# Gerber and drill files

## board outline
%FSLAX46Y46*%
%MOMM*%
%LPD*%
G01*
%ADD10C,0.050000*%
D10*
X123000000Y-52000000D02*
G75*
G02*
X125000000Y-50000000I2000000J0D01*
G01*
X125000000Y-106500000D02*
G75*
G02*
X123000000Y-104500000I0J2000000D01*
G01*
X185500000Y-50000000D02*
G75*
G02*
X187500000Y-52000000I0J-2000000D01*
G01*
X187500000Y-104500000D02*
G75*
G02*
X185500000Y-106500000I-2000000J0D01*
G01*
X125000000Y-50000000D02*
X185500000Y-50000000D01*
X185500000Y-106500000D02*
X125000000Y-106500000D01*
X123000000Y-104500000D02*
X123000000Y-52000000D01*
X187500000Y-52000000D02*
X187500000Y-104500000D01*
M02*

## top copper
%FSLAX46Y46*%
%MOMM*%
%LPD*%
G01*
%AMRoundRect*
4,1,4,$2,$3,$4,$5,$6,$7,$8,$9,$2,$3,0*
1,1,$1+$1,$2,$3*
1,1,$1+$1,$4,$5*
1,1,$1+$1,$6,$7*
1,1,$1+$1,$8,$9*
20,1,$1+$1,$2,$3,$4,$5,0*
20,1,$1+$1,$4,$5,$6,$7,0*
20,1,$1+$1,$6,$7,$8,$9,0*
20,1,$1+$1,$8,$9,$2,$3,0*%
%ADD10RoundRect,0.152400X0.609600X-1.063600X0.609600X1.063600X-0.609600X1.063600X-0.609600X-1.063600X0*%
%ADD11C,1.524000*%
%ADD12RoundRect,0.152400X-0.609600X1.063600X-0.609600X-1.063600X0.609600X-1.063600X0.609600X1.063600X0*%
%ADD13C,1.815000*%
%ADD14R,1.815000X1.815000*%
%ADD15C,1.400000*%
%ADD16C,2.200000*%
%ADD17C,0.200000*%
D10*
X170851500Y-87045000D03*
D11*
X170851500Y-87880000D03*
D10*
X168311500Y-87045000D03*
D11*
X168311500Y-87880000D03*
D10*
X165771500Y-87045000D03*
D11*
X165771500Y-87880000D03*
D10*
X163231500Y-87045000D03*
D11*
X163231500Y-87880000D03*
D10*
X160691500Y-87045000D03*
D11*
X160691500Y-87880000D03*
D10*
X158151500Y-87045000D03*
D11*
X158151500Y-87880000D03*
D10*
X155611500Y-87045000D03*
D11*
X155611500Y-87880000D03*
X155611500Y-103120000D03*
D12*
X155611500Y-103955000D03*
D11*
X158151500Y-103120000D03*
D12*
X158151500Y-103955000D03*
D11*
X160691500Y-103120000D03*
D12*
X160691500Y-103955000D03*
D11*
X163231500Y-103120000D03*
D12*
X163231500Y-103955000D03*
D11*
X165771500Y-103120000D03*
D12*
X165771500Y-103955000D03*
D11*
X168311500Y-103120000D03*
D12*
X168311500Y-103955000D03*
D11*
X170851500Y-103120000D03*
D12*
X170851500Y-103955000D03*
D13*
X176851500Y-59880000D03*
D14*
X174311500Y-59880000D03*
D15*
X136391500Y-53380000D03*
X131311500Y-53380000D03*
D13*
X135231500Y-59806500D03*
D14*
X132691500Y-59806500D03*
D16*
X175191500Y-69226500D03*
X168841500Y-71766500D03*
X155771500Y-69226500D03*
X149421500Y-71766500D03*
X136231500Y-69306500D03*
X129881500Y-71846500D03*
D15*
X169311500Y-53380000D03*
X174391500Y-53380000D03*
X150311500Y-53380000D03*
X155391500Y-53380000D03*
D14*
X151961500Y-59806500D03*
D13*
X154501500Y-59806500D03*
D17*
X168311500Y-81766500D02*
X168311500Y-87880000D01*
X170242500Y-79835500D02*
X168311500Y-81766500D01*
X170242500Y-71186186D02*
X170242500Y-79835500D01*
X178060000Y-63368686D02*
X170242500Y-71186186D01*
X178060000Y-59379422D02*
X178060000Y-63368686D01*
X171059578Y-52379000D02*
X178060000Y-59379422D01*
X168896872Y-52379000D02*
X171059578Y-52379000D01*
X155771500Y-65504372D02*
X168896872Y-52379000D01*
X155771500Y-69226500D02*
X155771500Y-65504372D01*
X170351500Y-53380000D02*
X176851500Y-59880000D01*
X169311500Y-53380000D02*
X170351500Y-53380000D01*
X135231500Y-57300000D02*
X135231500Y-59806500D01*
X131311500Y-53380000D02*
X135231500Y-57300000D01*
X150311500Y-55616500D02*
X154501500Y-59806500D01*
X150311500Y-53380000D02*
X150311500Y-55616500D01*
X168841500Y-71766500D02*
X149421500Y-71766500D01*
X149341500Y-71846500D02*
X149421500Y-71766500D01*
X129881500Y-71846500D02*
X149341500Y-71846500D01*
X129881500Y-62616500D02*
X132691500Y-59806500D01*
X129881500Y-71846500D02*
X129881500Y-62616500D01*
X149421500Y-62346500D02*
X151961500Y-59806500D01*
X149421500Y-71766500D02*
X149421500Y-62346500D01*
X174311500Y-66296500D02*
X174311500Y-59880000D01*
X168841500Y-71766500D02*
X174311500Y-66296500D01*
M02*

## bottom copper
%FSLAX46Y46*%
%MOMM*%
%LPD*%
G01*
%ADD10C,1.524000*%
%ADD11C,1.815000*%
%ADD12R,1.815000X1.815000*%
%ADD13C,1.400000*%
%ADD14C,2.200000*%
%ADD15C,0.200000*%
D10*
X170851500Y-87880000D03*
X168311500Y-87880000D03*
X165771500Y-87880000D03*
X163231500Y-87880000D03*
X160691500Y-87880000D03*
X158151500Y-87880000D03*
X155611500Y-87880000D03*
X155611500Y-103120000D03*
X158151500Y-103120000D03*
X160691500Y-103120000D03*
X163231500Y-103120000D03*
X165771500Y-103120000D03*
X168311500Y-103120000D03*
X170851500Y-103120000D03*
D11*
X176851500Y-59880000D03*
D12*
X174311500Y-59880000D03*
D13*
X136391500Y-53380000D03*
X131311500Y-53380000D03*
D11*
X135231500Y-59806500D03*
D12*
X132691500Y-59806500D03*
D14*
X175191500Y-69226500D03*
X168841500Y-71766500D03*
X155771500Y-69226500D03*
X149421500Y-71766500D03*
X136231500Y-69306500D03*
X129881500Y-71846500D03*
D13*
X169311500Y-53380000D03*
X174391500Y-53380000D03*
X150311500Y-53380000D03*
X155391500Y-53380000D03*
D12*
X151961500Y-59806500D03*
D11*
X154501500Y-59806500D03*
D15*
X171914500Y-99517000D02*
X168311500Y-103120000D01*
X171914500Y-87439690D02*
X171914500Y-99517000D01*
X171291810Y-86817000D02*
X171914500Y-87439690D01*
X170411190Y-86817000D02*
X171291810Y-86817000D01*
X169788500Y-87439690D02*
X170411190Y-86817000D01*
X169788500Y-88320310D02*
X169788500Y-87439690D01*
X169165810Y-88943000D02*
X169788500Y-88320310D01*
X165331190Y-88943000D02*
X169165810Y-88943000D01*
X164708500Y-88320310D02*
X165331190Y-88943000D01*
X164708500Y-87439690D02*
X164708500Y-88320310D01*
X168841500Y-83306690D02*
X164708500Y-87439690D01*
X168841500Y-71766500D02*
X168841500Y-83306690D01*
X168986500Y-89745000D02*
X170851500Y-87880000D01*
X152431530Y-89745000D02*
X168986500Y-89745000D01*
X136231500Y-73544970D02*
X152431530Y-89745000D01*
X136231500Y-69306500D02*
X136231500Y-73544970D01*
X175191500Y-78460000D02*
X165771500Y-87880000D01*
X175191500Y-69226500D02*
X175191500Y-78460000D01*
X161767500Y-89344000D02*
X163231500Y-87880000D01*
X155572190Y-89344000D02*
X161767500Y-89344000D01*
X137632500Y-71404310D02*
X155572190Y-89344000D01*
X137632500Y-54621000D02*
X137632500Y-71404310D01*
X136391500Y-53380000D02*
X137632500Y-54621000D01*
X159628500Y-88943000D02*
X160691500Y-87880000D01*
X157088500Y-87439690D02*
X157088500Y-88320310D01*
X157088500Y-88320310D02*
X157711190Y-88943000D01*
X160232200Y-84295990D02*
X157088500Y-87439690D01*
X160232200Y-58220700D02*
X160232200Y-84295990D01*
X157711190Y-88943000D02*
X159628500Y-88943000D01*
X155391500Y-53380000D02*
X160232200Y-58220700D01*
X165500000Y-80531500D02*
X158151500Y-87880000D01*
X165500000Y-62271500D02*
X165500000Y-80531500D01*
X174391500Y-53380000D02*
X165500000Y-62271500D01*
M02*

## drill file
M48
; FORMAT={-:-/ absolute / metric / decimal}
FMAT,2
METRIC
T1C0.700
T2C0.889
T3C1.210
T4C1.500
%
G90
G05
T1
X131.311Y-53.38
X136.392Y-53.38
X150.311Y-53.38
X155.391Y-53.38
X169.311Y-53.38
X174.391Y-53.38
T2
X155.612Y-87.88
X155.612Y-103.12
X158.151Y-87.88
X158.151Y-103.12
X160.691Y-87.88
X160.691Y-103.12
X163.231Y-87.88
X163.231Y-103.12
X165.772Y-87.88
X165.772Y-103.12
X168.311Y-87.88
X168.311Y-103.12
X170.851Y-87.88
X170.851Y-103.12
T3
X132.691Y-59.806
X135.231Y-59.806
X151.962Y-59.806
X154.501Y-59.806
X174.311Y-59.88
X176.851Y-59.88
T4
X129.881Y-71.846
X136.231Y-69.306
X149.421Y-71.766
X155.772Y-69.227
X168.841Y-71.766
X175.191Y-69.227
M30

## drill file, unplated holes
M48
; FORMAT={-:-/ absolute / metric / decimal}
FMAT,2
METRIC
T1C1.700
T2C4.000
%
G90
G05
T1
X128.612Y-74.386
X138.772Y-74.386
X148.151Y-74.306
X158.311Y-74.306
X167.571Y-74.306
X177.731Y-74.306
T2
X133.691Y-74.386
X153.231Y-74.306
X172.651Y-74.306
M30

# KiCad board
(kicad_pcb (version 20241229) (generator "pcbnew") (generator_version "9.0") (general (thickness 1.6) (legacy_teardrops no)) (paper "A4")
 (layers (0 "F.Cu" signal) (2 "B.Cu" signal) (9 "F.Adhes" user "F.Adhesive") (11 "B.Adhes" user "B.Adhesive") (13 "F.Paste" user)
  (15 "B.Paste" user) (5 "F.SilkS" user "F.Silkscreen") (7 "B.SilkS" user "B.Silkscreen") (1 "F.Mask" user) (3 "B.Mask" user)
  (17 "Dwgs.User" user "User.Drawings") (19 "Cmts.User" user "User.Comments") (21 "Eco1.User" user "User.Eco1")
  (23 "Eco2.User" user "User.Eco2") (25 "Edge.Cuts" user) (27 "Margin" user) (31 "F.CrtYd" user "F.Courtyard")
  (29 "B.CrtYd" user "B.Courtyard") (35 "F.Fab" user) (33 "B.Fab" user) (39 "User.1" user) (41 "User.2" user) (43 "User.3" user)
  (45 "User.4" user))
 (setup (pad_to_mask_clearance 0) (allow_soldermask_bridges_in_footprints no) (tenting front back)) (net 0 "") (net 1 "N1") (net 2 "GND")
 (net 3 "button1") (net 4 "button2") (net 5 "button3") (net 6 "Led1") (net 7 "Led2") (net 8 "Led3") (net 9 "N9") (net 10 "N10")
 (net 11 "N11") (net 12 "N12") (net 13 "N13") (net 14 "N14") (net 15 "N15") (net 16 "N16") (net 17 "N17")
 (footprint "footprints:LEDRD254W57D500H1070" (layer "F.Cu") (at 133.9615 59.8065)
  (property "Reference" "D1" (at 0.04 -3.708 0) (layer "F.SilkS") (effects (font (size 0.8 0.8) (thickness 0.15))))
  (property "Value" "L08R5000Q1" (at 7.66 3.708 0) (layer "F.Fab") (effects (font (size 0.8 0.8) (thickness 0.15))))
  (pad "A" thru_hole circle (at 1.27 0) (size 1.815 1.815) (drill 1.21) (layers "*.Cu" "*.Mask") (remove_unused_layers no) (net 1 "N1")
   (solder_mask_margin 0.102))
  (pad "C" thru_hole rect (at -1.27 0) (size 1.815 1.815) (drill 1.21) (layers "*.Cu" "*.Mask") (remove_unused_layers no) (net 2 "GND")
   (solder_mask_margin 0.102)))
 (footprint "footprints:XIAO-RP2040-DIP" (layer "F.Cu") (at 163.2315 95.5 -90)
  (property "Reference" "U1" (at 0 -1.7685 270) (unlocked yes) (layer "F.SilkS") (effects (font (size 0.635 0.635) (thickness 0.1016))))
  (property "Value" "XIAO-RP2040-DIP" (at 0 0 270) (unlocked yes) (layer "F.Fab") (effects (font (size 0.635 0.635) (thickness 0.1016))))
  (pad "1" smd roundrect (at -8.455 -7.62 90) (size 2.432 1.524) (layers "F.Cu" "F.Mask") (roundrect_rratio 0.1) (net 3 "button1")
   (thermal_bridge_angle 45))
  (pad "1" thru_hole circle (at -7.62 -7.62 90) (size 1.524 1.524) (drill 0.889) (layers "*.Cu" "*.Mask") (remove_unused_layers no)
   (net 3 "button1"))
  (pad "2" smd roundrect (at -8.455 -5.08 90) (size 2.432 1.524) (layers "F.Cu" "F.Mask") (roundrect_rratio 0.1) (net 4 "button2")
   (thermal_bridge_angle 45))
  (pad "2" thru_hole circle (at -7.62 -5.08 90) (size 1.524 1.524) (drill 0.889) (layers "*.Cu" "*.Mask") (remove_unused_layers no)
   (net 4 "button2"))
  (pad "3" smd roundrect (at -8.455 -2.54 90) (size 2.432 1.524) (layers "F.Cu" "F.Mask") (roundrect_rratio 0.1) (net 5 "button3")
   (thermal_bridge_angle 45))
  (pad "3" thru_hole circle (at -7.62 -2.54 90) (size 1.524 1.524) (drill 0.889) (layers "*.Cu" "*.Mask") (remove_unused_layers no)
   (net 5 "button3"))
  (pad "4" smd roundrect (at -8.455 0 90) (size 2.432 1.524) (layers "F.Cu" "F.Mask") (roundrect_rratio 0.1) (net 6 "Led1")
   (thermal_bridge_angle 45))
  (pad "4" thru_hole circle (at -7.62 0 90) (size 1.524 1.524) (drill 0.889) (layers "*.Cu" "*.Mask") (remove_unused_layers no)
   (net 6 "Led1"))
  (pad "5" smd roundrect (at -8.455 2.54 90) (size 2.432 1.524) (layers "F.Cu" "F.Mask") (roundrect_rratio 0.1) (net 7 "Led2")
   (thermal_bridge_angle 45))
  (pad "5" thru_hole circle (at -7.62 2.54 90) (size 1.524 1.524) (drill 0.889) (layers "*.Cu" "*.Mask") (remove_unused_layers no)
   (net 7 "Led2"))
  (pad "6" smd roundrect (at -8.455 5.08 90) (size 2.432 1.524) (layers "F.Cu" "F.Mask") (roundrect_rratio 0.1) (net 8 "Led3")
   (thermal_bridge_angle 45))
  (pad "6" thru_hole circle (at -7.62 5.08 90) (size 1.524 1.524) (drill 0.889) (layers "*.Cu" "*.Mask") (remove_unused_layers no)
   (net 8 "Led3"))
  (pad "7" smd roundrect (at -8.455 7.62 90) (size 2.432 1.524) (layers "F.Cu" "F.Mask") (roundrect_rratio 0.1) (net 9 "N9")
   (thermal_bridge_angle 45))
  (pad "7" thru_hole circle (at -7.62 7.62 90) (size 1.524 1.524) (drill 0.889) (layers "*.Cu" "*.Mask") (remove_unused_layers no)
   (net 9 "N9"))
  (pad "8" thru_hole circle (at 7.62 7.62 270) (size 1.524 1.524) (drill 0.889) (layers "*.Cu" "*.Mask") (remove_unused_layers no)
   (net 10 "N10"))
  (pad "8" smd roundrect (at 8.455 7.62 270) (size 2.432 1.524) (layers "F.Cu" "F.Mask") (roundrect_rratio 0.1) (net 10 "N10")
   (thermal_bridge_angle 45))
  (pad "9" thru_hole circle (at 7.62 5.08 270) (size 1.524 1.524) (drill 0.889) (layers "*.Cu" "*.Mask") (remove_unused_layers no)
   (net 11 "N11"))
  (pad "9" smd roundrect (at 8.455 5.08 270) (size 2.432 1.524) (layers "F.Cu" "F.Mask") (roundrect_rratio 0.1) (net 11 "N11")
   (thermal_bridge_angle 45))
  (pad "10" thru_hole circle (at 7.62 2.54 270) (size 1.524 1.524) (drill 0.889) (layers "*.Cu" "*.Mask") (remove_unused_layers no)
   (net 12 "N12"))
  (pad "10" smd roundrect (at 8.455 2.54 270) (size 2.432 1.524) (layers "F.Cu" "F.Mask") (roundrect_rratio 0.1) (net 12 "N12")
   (thermal_bridge_angle 45))
  (pad "11" thru_hole circle (at 7.62 0 270) (size 1.524 1.524) (drill 0.889) (layers "*.Cu" "*.Mask") (remove_unused_layers no)
   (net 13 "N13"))
  (pad "11" smd roundrect (at 8.455 0 270) (size 2.432 1.524) (layers "F.Cu" "F.Mask") (roundrect_rratio 0.1) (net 13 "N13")
   (thermal_bridge_angle 45))
  (pad "12" thru_hole circle (at 7.62 -2.54 270) (size 1.524 1.524) (drill 0.889) (layers "*.Cu" "*.Mask") (remove_unused_layers no)
   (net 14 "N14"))
  (pad "12" smd roundrect (at 8.455 -2.54 270) (size 2.432 1.524) (layers "F.Cu" "F.Mask") (roundrect_rratio 0.1) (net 14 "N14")
   (thermal_bridge_angle 45))
  (pad "13" thru_hole circle (at 7.62 -5.08 270) (size 1.524 1.524) (drill 0.889) (layers "*.Cu" "*.Mask") (remove_unused_layers no)
   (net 2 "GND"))
  (pad "13" smd roundrect (at 8.455 -5.08 270) (size 2.432 1.524) (layers "F.Cu" "F.Mask") (roundrect_rratio 0.1) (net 2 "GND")
   (thermal_bridge_angle 45))
  (pad "14" thru_hole circle (at 7.62 -7.62 270) (size 1.524 1.524) (drill 0.889) (layers "*.Cu" "*.Mask") (remove_unused_layers no)
   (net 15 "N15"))
  (pad "14" smd roundrect (at 8.455 -7.62 270) (size 2.432 1.524) (layers "F.Cu" "F.Mask") (roundrect_rratio 0.1) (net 15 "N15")
   (thermal_bridge_angle 45)))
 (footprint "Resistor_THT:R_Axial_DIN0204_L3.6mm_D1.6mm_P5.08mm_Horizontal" (layer "F.Cu") (at 169.3115 53.38)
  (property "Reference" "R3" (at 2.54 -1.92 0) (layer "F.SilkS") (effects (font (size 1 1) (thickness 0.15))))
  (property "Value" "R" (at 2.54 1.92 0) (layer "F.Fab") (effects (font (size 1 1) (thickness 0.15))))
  (pad "1" thru_hole circle (at 0 0) (size 1.4 1.4) (drill 0.7) (layers "*.Cu" "*.Mask") (remove_unused_layers no) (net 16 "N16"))
  (pad "2" thru_hole circle (at 5.08 0) (size 1.4 1.4) (drill 0.7) (layers "*.Cu" "*.Mask") (remove_unused_layers no) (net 8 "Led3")))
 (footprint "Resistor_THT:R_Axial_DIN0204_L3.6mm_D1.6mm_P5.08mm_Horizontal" (layer "F.Cu") (at 131.3115 53.38)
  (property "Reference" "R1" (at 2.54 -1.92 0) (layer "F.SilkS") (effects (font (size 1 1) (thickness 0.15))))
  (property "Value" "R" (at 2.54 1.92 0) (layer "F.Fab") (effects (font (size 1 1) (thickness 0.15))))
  (pad "1" thru_hole circle (at 0 0) (size 1.4 1.4) (drill 0.7) (layers "*.Cu" "*.Mask") (remove_unused_layers no) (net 1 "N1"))
  (pad "2" thru_hole circle (at 5.08 0) (size 1.4 1.4) (drill 0.7) (layers "*.Cu" "*.Mask") (remove_unused_layers no) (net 6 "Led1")))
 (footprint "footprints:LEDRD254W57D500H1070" (layer "F.Cu") (at 153.2315 59.8065)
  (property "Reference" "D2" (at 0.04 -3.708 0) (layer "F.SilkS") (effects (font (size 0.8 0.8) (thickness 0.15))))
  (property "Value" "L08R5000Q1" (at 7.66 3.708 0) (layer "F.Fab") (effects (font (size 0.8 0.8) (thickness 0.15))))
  (pad "A" thru_hole circle (at 1.27 0) (size 1.815 1.815) (drill 1.21) (layers "*.Cu" "*.Mask") (remove_unused_layers no) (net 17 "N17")
   (solder_mask_margin 0.102))
  (pad "C" thru_hole rect (at -1.27 0) (size 1.815 1.815) (drill 1.21) (layers "*.Cu" "*.Mask") (remove_unused_layers no) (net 2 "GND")
   (solder_mask_margin 0.102)))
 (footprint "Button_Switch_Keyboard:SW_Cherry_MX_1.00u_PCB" (layer "F.Cu") (at 155.7715 69.2265)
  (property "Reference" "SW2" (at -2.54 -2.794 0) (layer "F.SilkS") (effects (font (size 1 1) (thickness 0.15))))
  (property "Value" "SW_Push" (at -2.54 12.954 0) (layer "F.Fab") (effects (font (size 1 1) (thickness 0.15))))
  (pad "" np_thru_hole circle (at -7.62 5.08) (size 1.7 1.7) (drill 1.7) (layers "*.Cu" "*.Mask"))
  (pad "" np_thru_hole circle (at -2.54 5.08) (size 4 4) (drill 4) (layers "*.Cu" "*.Mask"))
  (pad "" np_thru_hole circle (at 2.54 5.08) (size 1.7 1.7) (drill 1.7) (layers "*.Cu" "*.Mask"))
  (pad "1" thru_hole circle (at 0 0) (size 2.2 2.2) (drill 1.5) (layers "*.Cu" "*.Mask") (remove_unused_layers no) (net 4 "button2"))
  (pad "2" thru_hole circle (at -6.35 2.54) (size 2.2 2.2) (drill 1.5) (layers "*.Cu" "*.Mask") (remove_unused_layers no) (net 2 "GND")))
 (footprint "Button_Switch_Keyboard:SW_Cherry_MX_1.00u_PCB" (layer "F.Cu") (at 136.2315 69.3065)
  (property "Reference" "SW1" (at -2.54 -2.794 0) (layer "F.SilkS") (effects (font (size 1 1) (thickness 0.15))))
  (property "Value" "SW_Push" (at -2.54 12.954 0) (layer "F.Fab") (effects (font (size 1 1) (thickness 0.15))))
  (pad "" np_thru_hole circle (at -7.62 5.08) (size 1.7 1.7) (drill 1.7) (layers "*.Cu" "*.Mask"))
  (pad "" np_thru_hole circle (at -2.54 5.08) (size 4 4) (drill 4) (layers "*.Cu" "*.Mask"))
  (pad "" np_thru_hole circle (at 2.54 5.08) (size 1.7 1.7) (drill 1.7) (layers "*.Cu" "*.Mask"))
  (pad "1" thru_hole circle (at 0 0) (size 2.2 2.2) (drill 1.5) (layers "*.Cu" "*.Mask") (remove_unused_layers no) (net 3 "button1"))
  (pad "2" thru_hole circle (at -6.35 2.54) (size 2.2 2.2) (drill 1.5) (layers "*.Cu" "*.Mask") (remove_unused_layers no) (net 2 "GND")))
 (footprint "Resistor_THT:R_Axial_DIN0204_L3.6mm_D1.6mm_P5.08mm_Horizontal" (layer "F.Cu") (at 150.3115 53.38)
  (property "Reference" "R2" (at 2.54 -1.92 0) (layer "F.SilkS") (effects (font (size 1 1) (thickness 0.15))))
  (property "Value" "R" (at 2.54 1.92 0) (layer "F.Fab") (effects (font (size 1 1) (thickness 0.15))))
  (pad "1" thru_hole circle (at 0 0) (size 1.4 1.4) (drill 0.7) (layers "*.Cu" "*.Mask") (remove_unused_layers no) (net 17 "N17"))
  (pad "2" thru_hole circle (at 5.08 0) (size 1.4 1.4) (drill 0.7) (layers "*.Cu" "*.Mask") (remove_unused_layers no) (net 7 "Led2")))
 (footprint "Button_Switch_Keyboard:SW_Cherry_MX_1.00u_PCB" (layer "F.Cu") (at 175.1915 69.2265)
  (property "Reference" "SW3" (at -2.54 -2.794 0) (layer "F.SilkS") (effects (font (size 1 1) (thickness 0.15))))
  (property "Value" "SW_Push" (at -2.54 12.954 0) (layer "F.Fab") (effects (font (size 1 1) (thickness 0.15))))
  (pad "" np_thru_hole circle (at -7.62 5.08) (size 1.7 1.7) (drill 1.7) (layers "*.Cu" "*.Mask"))
  (pad "" np_thru_hole circle (at -2.54 5.08) (size 4 4) (drill 4) (layers "*.Cu" "*.Mask"))
  (pad "" np_thru_hole circle (at 2.54 5.08) (size 1.7 1.7) (drill 1.7) (layers "*.Cu" "*.Mask"))
  (pad "1" thru_hole circle (at 0 0) (size 2.2 2.2) (drill 1.5) (layers "*.Cu" "*.Mask") (remove_unused_layers no) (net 5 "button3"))
  (pad "2" thru_hole circle (at -6.35 2.54) (size 2.2 2.2) (drill 1.5) (layers "*.Cu" "*.Mask") (remove_unused_layers no) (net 2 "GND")))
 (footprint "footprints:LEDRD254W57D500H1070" (layer "F.Cu") (at 175.5815 59.88)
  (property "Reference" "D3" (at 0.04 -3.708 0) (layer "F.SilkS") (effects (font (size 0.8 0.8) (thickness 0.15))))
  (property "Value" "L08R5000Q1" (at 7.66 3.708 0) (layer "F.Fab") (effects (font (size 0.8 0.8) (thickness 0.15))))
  (pad "A" thru_hole circle (at 1.27 0) (size 1.815 1.815) (drill 1.21) (layers "*.Cu" "*.Mask") (remove_unused_layers no) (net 16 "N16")
   (solder_mask_margin 0.102))
  (pad "C" thru_hole rect (at -1.27 0) (size 1.815 1.815) (drill 1.21) (layers "*.Cu" "*.Mask") (remove_unused_layers no) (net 2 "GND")
   (solder_mask_margin 0.102)))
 (gr_arc (start 123 52) (mid 123.585786 50.585786) (end 125 50) (stroke (width 0.05) (type default)) (layer "Edge.Cuts"))
 (gr_line (start 187.5 52) (end 187.5 104.5) (stroke (width 0.05) (type default)) (layer "Edge.Cuts"))
 (gr_arc (start 187.5 104.5) (mid 186.914214 105.914214) (end 185.5 106.5) (stroke (width 0.05) (type default)) (layer "Edge.Cuts"))
 (gr_arc (start 125 106.5) (mid 123.585786 105.914214) (end 123 104.5) (stroke (width 0.05) (type default)) (layer "Edge.Cuts"))
 (gr_line (start 123 104.5) (end 123 52) (stroke (width 0.05) (type default)) (layer "Edge.Cuts"))
 (gr_line (start 125 50) (end 185.5 50) (stroke (width 0.05) (type default)) (layer "Edge.Cuts"))
 (gr_arc (start 185.5 50) (mid 186.914214 50.585786) (end 187.5 52) (stroke (width 0.05) (type default)) (layer "Edge.Cuts"))
 (gr_line (start 185.5 106.5) (end 125 106.5) (stroke (width 0.05) (type default)) (layer "Edge.Cuts"))
 (segment (start 168.8415 71.7665) (end 149.4215 71.7665) (width 0.2) (layer "F.Cu") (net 2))
 (segment (start 149.4215 62.3465) (end 151.9615 59.8065) (width 0.2) (layer "F.Cu") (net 2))
 (segment (start 149.3415 71.8465) (end 149.4215 71.7665) (width 0.2) (layer "F.Cu") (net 2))
 (segment (start 149.4215 71.7665) (end 149.4215 62.3465) (width 0.2) (layer "F.Cu") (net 2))
 (segment (start 168.8415 71.7665) (end 174.3115 66.2965) (width 0.2) (layer "F.Cu") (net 2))
 (segment (start 129.8815 71.8465) (end 129.8815 62.6165) (width 0.2) (layer "F.Cu") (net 2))
 (segment (start 129.8815 71.8465) (end 149.3415 71.8465) (width 0.2) (layer "F.Cu") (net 2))
 (segment (start 129.8815 62.6165) (end 132.6915 59.8065) (width 0.2) (layer "F.Cu") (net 2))
 (segment (start 174.3115 66.2965) (end 174.3115 59.88) (width 0.2) (layer "F.Cu") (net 2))
 (segment (start 171.9145 99.517) (end 168.3115 103.12) (width 0.2) (layer "B.Cu") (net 2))
 (segment (start 171.9145 87.43969) (end 171.9145 99.517) (width 0.2) (layer "B.Cu") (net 2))
 (segment (start 170.41119 86.817) (end 171.29181 86.817) (width 0.2) (layer "B.Cu") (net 2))
 (segment (start 169.7885 87.43969) (end 170.41119 86.817) (width 0.2) (layer "B.Cu") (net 2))
 (segment (start 169.16581 88.943) (end 169.7885 88.32031) (width 0.2) (layer "B.Cu") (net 2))
 (segment (start 171.29181 86.817) (end 171.9145 87.43969) (width 0.2) (layer "B.Cu") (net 2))
 (segment (start 164.7085 87.43969) (end 164.7085 88.32031) (width 0.2) (layer "B.Cu") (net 2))
 (segment (start 168.8415 71.7665) (end 168.8415 83.30669) (width 0.2) (layer "B.Cu") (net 2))
 (segment (start 164.7085 88.32031) (end 165.33119 88.943) (width 0.2) (layer "B.Cu") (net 2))
 (segment (start 169.7885 88.32031) (end 169.7885 87.43969) (width 0.2) (layer "B.Cu") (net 2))
 (segment (start 168.8415 83.30669) (end 164.7085 87.43969) (width 0.2) (layer "B.Cu") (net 2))
 (segment (start 165.33119 88.943) (end 169.16581 88.943) (width 0.2) (layer "B.Cu") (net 2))
 (segment (start 135.2315 57.3) (end 135.2315 59.8065) (width 0.2) (layer "F.Cu") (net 1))
 (segment (start 131.3115 53.38) (end 135.2315 57.3) (width 0.2) (layer "F.Cu") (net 1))
 (segment (start 150.3115 55.6165) (end 154.5015 59.8065) (width 0.2) (layer "F.Cu") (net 17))
 (segment (start 150.3115 53.38) (end 150.3115 55.6165) (width 0.2) (layer "F.Cu") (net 17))
 (segment (start 170.3515 53.38) (end 176.8515 59.88) (width 0.2) (layer "F.Cu") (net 16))
 (segment (start 169.3115 53.38) (end 170.3515 53.38) (width 0.2) (layer "F.Cu") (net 16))
 (segment (start 155.57219 89.344) (end 161.7675 89.344) (width 0.2) (layer "B.Cu") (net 6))
 (segment (start 136.3915 53.38) (end 137.6325 54.621) (width 0.2) (layer "B.Cu") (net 6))
 (segment (start 137.6325 71.40431) (end 155.57219 89.344) (width 0.2) (layer "B.Cu") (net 6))
 (segment (start 161.7675 89.344) (end 163.2315 87.88) (width 0.2) (layer "B.Cu") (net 6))
 (segment (start 137.6325 54.621) (end 137.6325 71.40431) (width 0.2) (layer "B.Cu") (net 6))
 (segment (start 157.0885 88.32031) (end 157.71119 88.943) (width 0.2) (layer "B.Cu") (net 7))
 (segment (start 157.0885 87.43969) (end 157.0885 88.32031) (width 0.2) (layer "B.Cu") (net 7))
 (segment (start 160.2322 84.29599) (end 157.0885 87.43969) (width 0.2) (layer "B.Cu") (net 7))
 (segment (start 159.6285 88.943) (end 160.6915 87.88) (width 0.2) (layer "B.Cu") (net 7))
 (segment (start 155.3915 53.38) (end 160.2322 58.2207) (width 0.2) (layer "B.Cu") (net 7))
 (segment (start 157.71119 88.943) (end 159.6285 88.943) (width 0.2) (layer "B.Cu") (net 7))
 (segment (start 160.2322 58.2207) (end 160.2322 84.29599) (width 0.2) (layer "B.Cu") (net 7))
 (segment (start 174.3915 53.38) (end 165.5 62.2715) (width 0.2) (layer "B.Cu") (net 8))
 (segment (start 165.5 80.5315) (end 158.1515 87.88) (width 0.2) (layer "B.Cu") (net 8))
 (segment (start 165.5 62.2715) (end 165.5 80.5315) (width 0.2) (layer "B.Cu") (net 8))
 (segment (start 152.43153 89.745) (end 168.9865 89.745) (width 0.2) (layer "B.Cu") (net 3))
 (segment (start 136.2315 69.3065) (end 136.2315 73.54497) (width 0.2) (layer "B.Cu") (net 3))
 (segment (start 136.2315 73.54497) (end 152.43153 89.745) (width 0.2) (layer "B.Cu") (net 3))
 (segment (start 168.9865 89.745) (end 170.8515 87.88) (width 0.2) (layer "B.Cu") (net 3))
 (segment (start 178.06 59.379422) (end 178.06 63.368686) (width 0.2) (layer "F.Cu") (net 4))
 (segment (start 155.7715 65.504372) (end 168.896872 52.379) (width 0.2) (layer "F.Cu") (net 4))
 (segment (start 170.2425 71.186186) (end 170.2425 79.8355) (width 0.2) (layer "F.Cu") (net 4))
 (segment (start 178.06 63.368686) (end 170.2425 71.186186) (width 0.2) (layer "F.Cu") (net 4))
 (segment (start 168.3115 81.7665) (end 168.3115 87.88) (width 0.2) (layer "F.Cu") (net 4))
 (segment (start 170.2425 79.8355) (end 168.3115 81.7665) (width 0.2) (layer "F.Cu") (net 4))
 (segment (start 168.896872 52.379) (end 171.059578 52.379) (width 0.2) (layer "F.Cu") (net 4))
 (segment (start 155.7715 69.2265) (end 155.7715 65.504372) (width 0.2) (layer "F.Cu") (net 4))
 (segment (start 171.059578 52.379) (end 178.06 59.379422) (width 0.2) (layer "F.Cu") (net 4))
 (segment (start 175.1915 69.2265) (end 175.1915 78.46) (width 0.2) (layer "B.Cu") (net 5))
 (segment (start 175.1915 78.46) (end 165.7715 87.88) (width 0.2) (layer "B.Cu") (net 5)))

